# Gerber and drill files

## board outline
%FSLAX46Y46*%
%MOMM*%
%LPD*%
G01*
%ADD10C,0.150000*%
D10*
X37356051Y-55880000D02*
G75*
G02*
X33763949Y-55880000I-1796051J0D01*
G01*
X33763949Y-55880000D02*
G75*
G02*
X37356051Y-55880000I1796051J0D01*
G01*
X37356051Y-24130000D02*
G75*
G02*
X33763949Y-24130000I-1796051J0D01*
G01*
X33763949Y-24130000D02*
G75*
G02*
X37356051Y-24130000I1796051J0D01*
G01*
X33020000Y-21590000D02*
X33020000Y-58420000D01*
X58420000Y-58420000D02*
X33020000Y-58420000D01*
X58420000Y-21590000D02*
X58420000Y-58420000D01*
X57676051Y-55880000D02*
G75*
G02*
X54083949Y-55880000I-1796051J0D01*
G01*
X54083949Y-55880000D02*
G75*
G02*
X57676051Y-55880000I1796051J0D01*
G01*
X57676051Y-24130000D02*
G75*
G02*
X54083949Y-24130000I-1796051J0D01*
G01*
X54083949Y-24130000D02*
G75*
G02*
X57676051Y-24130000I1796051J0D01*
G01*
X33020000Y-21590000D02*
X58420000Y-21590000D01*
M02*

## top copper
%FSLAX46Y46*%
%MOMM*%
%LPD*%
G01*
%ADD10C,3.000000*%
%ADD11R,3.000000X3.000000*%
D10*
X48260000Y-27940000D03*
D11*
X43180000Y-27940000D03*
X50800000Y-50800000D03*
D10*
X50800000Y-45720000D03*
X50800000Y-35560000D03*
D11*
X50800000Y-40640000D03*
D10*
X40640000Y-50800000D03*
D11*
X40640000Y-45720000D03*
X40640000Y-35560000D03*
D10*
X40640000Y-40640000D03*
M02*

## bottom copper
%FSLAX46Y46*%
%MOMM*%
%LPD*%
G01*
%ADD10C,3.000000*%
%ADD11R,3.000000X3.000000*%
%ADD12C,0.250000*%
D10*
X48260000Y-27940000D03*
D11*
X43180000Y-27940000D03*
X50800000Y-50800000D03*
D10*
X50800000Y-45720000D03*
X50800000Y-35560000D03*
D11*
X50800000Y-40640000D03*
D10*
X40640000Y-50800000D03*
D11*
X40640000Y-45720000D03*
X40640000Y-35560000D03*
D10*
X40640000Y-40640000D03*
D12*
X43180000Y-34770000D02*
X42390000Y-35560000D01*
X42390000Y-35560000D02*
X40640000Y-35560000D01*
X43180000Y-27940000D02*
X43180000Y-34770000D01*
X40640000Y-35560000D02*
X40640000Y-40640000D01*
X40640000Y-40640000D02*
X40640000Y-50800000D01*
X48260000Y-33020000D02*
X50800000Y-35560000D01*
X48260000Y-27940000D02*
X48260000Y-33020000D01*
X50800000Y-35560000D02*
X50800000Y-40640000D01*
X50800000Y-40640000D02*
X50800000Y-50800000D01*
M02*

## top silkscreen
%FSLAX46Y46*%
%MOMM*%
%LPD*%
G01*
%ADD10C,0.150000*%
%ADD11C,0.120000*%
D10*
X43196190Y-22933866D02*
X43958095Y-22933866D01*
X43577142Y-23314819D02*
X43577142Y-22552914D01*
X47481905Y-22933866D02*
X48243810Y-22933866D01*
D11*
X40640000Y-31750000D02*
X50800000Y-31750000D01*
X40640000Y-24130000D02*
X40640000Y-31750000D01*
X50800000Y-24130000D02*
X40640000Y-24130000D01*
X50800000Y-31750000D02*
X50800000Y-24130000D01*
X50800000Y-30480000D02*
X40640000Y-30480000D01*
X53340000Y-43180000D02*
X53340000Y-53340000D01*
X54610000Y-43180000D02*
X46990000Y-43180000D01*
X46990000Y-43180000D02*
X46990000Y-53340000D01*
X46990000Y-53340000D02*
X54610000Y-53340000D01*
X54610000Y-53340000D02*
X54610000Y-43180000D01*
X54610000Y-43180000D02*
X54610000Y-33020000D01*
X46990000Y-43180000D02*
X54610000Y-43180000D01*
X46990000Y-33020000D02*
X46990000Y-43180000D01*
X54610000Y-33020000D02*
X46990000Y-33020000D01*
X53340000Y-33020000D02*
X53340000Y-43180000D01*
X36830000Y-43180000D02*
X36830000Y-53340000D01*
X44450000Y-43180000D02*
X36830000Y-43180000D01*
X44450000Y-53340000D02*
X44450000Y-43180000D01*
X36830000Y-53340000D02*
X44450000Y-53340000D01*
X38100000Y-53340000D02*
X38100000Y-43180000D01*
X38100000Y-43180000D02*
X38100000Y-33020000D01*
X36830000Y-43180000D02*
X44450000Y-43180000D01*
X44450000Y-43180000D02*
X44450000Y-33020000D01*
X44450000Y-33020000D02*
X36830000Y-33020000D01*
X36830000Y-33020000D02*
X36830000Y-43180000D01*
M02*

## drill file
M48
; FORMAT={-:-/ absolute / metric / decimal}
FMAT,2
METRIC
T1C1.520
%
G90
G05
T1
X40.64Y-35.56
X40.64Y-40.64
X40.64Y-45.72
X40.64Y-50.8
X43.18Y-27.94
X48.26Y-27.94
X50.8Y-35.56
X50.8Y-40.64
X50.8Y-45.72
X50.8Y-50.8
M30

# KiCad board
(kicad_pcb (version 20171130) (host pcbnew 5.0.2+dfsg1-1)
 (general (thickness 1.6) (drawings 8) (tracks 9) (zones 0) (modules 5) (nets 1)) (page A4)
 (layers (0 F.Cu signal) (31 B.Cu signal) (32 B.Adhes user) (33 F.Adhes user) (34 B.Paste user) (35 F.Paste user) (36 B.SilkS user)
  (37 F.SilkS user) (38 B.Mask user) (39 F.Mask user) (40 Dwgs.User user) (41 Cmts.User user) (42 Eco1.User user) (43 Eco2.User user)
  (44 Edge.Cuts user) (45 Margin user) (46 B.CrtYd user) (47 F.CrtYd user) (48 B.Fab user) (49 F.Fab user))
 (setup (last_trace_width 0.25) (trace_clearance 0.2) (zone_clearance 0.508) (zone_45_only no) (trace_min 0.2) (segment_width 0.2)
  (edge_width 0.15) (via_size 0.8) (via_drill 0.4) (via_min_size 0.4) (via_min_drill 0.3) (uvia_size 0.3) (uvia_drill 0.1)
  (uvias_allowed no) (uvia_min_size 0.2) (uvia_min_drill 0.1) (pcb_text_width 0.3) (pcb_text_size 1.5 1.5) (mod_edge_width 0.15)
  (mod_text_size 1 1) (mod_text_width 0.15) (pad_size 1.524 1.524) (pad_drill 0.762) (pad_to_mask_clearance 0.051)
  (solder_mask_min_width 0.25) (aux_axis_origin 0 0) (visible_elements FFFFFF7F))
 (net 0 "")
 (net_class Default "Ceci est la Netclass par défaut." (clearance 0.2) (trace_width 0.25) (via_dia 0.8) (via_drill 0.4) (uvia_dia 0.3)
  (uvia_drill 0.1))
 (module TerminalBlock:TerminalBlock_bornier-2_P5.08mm (layer F.Cu) (at 43.18 27.94)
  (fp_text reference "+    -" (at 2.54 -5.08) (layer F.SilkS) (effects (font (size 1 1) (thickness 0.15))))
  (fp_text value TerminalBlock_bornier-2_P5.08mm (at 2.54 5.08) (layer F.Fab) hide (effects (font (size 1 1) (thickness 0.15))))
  (fp_line (start -2.54 3.81) (end 7.62 3.81) (layer F.SilkS) (width 0.12))
  (fp_line (start -2.54 -3.81) (end -2.54 3.81) (layer F.SilkS) (width 0.12))
  (fp_line (start 7.62 -3.81) (end -2.54 -3.81) (layer F.SilkS) (width 0.12))
  (fp_line (start 7.62 3.81) (end 7.62 -3.81) (layer F.SilkS) (width 0.12))
  (fp_line (start 7.62 2.54) (end -2.54 2.54) (layer F.SilkS) (width 0.12))
  (pad 2 thru_hole circle (at 5.08 0) (size 3 3) (drill 1.52) (layers *.Cu *.Mask))
  (pad 1 thru_hole rect (at 0 0) (size 3 3) (drill 1.52) (layers *.Cu *.Mask)))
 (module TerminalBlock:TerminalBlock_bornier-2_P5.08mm (layer F.Cu) (at 50.8 50.8 90)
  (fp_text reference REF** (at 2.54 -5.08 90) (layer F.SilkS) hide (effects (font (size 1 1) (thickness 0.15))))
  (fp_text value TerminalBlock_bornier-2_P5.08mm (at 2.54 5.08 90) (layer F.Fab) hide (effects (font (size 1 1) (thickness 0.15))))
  (fp_line (start 7.62 2.54) (end -2.54 2.54) (layer F.SilkS) (width 0.12))
  (fp_line (start 7.62 3.81) (end 7.62 -3.81) (layer F.SilkS) (width 0.12))
  (fp_line (start 7.62 -3.81) (end -2.54 -3.81) (layer F.SilkS) (width 0.12))
  (fp_line (start -2.54 -3.81) (end -2.54 3.81) (layer F.SilkS) (width 0.12))
  (fp_line (start -2.54 3.81) (end 7.62 3.81) (layer F.SilkS) (width 0.12))
  (pad 1 thru_hole rect (at 0 0 90) (size 3 3) (drill 1.52) (layers *.Cu *.Mask))
  (pad 2 thru_hole circle (at 5.08 0 90) (size 3 3) (drill 1.52) (layers *.Cu *.Mask)))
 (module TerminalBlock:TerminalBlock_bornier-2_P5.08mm (layer F.Cu) (at 50.8 40.64 90)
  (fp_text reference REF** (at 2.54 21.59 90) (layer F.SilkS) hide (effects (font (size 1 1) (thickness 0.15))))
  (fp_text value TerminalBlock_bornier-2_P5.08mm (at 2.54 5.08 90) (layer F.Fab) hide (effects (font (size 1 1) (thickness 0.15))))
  (fp_line (start -2.54 3.81) (end 7.62 3.81) (layer F.SilkS) (width 0.12))
  (fp_line (start -2.54 -3.81) (end -2.54 3.81) (layer F.SilkS) (width 0.12))
  (fp_line (start 7.62 -3.81) (end -2.54 -3.81) (layer F.SilkS) (width 0.12))
  (fp_line (start 7.62 3.81) (end 7.62 -3.81) (layer F.SilkS) (width 0.12))
  (fp_line (start 7.62 2.54) (end -2.54 2.54) (layer F.SilkS) (width 0.12))
  (pad 2 thru_hole circle (at 5.08 0 90) (size 3 3) (drill 1.52) (layers *.Cu *.Mask))
  (pad 1 thru_hole rect (at 0 0 90) (size 3 3) (drill 1.52) (layers *.Cu *.Mask)))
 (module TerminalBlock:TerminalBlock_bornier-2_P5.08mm (layer F.Cu) (at 40.64 45.72 270)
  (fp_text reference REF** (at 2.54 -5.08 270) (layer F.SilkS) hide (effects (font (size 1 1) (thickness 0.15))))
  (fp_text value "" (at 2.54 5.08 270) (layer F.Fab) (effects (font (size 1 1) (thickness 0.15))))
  (fp_line (start -2.54 3.81) (end 7.62 3.81) (layer F.SilkS) (width 0.12))
  (fp_line (start -2.54 -3.81) (end -2.54 3.81) (layer F.SilkS) (width 0.12))
  (fp_line (start 7.62 -3.81) (end -2.54 -3.81) (layer F.SilkS) (width 0.12))
  (fp_line (start 7.62 3.81) (end 7.62 -3.81) (layer F.SilkS) (width 0.12))
  (fp_line (start 7.62 2.54) (end -2.54 2.54) (layer F.SilkS) (width 0.12))
  (pad 2 thru_hole circle (at 5.08 0 270) (size 3 3) (drill 1.52) (layers *.Cu *.Mask))
  (pad 1 thru_hole rect (at 0 0 270) (size 3 3) (drill 1.52) (layers *.Cu *.Mask)))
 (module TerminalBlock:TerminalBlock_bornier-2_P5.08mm (layer F.Cu) (at 40.64 35.56 270)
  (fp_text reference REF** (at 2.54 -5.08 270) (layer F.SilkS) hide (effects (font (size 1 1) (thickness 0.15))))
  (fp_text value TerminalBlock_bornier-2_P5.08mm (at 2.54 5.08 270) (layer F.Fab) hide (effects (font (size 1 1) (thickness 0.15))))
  (fp_line (start 7.62 2.54) (end -2.54 2.54) (layer F.SilkS) (width 0.12))
  (fp_line (start 7.62 3.81) (end 7.62 -3.81) (layer F.SilkS) (width 0.12))
  (fp_line (start 7.62 -3.81) (end -2.54 -3.81) (layer F.SilkS) (width 0.12))
  (fp_line (start -2.54 -3.81) (end -2.54 3.81) (layer F.SilkS) (width 0.12))
  (fp_line (start -2.54 3.81) (end 7.62 3.81) (layer F.SilkS) (width 0.12))
  (pad 1 thru_hole rect (at 0 0 270) (size 3 3) (drill 1.52) (layers *.Cu *.Mask))
  (pad 2 thru_hole circle (at 5.08 0 270) (size 3 3) (drill 1.52) (layers *.Cu *.Mask)))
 (gr_circle (center 35.56 55.88) (end 36.83 57.15) (layer Edge.Cuts) (width 0.15))
 (gr_circle (center 35.56 24.13) (end 36.83 25.4) (layer Edge.Cuts) (width 0.15))
 (gr_line (start 33.02 21.59) (end 33.02 58.42) (layer Edge.Cuts) (width 0.15))
 (gr_line (start 58.42 58.42) (end 33.02 58.42) (layer Edge.Cuts) (width 0.15))
 (gr_line (start 58.42 21.59) (end 58.42 58.42) (layer Edge.Cuts) (width 0.15))
 (gr_circle (center 55.88 55.88) (end 57.15 57.15) (layer Edge.Cuts) (width 0.15))
 (gr_circle (center 55.88 24.13) (end 57.15 25.4) (layer Edge.Cuts) (width 0.15))
 (gr_line (start 33.02 21.59) (end 58.42 21.59) (layer Edge.Cuts) (width 0.15))
 (segment (start 43.18 34.77) (end 42.39 35.56) (width 0.25) (layer B.Cu) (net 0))
 (segment (start 42.39 35.56) (end 40.64 35.56) (width 0.25) (layer B.Cu) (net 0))
 (segment (start 43.18 27.94) (end 43.18 34.77) (width 0.25) (layer B.Cu) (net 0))
 (segment (start 40.64 35.56) (end 40.64 40.64) (width 0.25) (layer B.Cu) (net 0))
 (segment (start 40.64 40.64) (end 40.64 50.8) (width 0.25) (layer B.Cu) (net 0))
 (segment (start 48.26 33.02) (end 50.8 35.56) (width 0.25) (layer B.Cu) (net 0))
 (segment (start 48.26 27.94) (end 48.26 33.02) (width 0.25) (layer B.Cu) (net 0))
 (segment (start 50.8 35.56) (end 50.8 40.64) (width 0.25) (layer B.Cu) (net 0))
 (segment (start 50.8 40.64) (end 50.8 50.8) (width 0.25) (layer B.Cu) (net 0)))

